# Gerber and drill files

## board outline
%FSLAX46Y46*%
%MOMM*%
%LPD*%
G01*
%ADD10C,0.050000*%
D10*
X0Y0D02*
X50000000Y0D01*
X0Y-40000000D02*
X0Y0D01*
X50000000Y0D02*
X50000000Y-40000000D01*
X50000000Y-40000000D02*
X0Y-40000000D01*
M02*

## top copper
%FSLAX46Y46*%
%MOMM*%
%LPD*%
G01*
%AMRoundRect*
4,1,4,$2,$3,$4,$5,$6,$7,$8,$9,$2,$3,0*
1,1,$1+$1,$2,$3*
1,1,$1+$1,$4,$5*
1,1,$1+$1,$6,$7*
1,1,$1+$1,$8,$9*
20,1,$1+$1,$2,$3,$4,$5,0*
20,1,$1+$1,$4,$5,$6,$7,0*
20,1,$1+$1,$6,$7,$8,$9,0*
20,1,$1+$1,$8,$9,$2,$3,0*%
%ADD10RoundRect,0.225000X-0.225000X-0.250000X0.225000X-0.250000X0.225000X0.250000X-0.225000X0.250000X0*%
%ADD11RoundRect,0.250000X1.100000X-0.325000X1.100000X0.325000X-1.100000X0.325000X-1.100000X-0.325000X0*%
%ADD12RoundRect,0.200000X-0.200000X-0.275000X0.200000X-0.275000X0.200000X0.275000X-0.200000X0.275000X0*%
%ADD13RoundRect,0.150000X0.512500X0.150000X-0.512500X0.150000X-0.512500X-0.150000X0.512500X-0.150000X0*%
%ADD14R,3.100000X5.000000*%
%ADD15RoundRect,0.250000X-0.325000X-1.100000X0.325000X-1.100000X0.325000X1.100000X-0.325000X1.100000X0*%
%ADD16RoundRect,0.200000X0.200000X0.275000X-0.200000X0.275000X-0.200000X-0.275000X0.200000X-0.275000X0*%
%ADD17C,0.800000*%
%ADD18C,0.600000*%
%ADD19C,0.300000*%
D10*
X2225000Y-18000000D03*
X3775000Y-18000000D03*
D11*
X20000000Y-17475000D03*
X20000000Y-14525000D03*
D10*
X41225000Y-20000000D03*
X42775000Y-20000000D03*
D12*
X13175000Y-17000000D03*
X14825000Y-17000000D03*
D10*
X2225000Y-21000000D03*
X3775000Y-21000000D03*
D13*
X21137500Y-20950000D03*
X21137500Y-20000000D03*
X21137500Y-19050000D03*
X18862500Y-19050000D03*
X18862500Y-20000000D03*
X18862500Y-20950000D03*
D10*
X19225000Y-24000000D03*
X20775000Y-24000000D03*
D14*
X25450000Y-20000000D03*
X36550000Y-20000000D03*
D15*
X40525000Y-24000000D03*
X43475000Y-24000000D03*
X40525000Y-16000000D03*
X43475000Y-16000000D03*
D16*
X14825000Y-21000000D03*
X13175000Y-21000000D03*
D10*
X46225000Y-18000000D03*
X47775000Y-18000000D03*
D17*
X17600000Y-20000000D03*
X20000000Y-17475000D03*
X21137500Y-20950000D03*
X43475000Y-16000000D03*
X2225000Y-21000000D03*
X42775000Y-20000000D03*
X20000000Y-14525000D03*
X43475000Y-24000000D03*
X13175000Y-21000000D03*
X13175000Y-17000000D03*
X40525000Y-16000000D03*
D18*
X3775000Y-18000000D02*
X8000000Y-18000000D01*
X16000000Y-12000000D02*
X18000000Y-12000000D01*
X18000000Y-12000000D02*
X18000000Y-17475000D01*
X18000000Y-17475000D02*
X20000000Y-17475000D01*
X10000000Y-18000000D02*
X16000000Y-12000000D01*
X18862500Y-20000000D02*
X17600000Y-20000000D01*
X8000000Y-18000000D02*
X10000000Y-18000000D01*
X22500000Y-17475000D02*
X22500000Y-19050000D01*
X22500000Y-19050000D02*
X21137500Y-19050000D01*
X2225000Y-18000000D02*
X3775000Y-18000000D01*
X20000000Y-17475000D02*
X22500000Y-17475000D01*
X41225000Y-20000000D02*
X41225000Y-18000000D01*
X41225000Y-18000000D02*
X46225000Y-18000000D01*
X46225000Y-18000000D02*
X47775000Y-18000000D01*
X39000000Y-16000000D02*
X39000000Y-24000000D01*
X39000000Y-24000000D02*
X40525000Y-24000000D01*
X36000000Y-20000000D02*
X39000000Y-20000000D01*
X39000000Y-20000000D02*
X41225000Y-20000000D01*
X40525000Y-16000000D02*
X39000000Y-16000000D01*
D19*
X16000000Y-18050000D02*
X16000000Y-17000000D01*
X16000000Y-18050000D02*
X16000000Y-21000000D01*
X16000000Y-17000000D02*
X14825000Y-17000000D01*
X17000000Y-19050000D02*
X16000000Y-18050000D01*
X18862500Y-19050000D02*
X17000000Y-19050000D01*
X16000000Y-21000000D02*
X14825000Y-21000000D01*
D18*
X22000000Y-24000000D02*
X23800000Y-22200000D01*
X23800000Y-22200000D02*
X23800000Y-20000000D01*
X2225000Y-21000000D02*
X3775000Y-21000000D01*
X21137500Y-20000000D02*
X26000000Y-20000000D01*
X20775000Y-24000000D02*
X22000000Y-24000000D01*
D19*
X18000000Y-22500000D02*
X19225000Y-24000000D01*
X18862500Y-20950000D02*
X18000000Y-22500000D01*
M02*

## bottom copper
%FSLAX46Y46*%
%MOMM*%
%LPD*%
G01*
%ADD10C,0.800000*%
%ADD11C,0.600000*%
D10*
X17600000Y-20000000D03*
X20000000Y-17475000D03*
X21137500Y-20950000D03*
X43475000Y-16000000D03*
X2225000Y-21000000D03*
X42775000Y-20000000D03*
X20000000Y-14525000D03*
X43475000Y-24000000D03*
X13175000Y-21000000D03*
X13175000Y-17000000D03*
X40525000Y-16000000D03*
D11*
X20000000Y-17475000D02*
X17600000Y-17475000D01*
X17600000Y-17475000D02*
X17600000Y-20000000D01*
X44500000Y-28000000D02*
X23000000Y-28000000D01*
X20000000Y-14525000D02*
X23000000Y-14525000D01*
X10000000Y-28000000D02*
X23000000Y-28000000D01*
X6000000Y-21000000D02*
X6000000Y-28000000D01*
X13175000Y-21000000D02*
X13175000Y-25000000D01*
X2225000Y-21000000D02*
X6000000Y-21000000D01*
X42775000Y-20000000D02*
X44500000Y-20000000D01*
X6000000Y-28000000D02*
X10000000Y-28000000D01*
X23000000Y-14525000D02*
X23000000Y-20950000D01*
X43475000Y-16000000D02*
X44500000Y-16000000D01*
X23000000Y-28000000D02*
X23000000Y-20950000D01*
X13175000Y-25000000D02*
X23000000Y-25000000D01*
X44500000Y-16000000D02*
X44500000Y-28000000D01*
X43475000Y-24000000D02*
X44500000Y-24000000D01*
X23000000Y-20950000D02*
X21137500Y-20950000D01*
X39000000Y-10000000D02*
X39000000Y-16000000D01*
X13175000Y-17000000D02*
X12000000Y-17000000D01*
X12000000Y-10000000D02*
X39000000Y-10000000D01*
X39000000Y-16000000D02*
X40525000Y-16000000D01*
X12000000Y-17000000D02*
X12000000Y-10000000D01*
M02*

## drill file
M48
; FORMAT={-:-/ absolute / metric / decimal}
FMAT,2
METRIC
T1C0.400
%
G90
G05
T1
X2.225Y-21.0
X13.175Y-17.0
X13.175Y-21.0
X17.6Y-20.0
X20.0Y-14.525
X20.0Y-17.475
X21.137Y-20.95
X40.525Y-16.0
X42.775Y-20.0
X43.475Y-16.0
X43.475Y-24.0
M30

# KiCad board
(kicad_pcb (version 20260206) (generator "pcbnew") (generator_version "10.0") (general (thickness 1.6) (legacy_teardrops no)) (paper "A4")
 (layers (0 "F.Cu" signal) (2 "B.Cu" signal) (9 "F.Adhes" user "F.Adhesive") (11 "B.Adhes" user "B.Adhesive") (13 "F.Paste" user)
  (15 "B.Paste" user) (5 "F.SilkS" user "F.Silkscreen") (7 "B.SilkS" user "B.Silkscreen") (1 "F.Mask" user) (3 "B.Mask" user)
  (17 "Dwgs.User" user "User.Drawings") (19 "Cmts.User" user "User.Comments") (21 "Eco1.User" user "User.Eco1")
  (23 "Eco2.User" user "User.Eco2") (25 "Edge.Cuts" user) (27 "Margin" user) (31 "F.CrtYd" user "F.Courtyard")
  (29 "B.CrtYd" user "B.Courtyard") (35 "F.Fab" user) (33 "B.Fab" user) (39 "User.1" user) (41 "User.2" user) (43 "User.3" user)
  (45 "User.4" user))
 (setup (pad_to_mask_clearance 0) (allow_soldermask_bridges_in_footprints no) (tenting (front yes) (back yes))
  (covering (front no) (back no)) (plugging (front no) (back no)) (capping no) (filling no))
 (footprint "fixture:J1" (layer "F.Cu") (at 3 18)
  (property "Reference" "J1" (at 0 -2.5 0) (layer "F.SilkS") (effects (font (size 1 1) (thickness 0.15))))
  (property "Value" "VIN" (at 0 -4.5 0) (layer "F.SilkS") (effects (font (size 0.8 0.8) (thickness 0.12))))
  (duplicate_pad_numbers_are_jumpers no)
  (pad "1" smd roundrect (at -0.775 0) (size 0.9 0.95) (layers "F.Cu" "F.Mask" "F.Paste") (roundrect_rratio 0.25) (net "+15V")
   (thermal_bridge_angle 45))
  (pad "2" smd roundrect (at 0.775 0) (size 0.9 0.95) (layers "F.Cu" "F.Mask" "F.Paste") (roundrect_rratio 0.25) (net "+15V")
   (thermal_bridge_angle 45)))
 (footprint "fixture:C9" (layer "F.Cu") (at 20 16 90)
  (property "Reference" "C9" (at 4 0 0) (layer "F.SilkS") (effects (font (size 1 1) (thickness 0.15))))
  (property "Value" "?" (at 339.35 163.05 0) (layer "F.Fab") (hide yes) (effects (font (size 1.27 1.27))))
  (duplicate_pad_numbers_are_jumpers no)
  (pad "1" smd roundrect (at -1.475 0 90) (size 1.15 2.7) (layers "F.Cu" "F.Mask" "F.Paste") (roundrect_rratio 0.217391) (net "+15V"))
  (pad "2" smd roundrect (at 1.475 0 90) (size 1.15 2.7) (layers "F.Cu" "F.Mask" "F.Paste") (roundrect_rratio 0.217391) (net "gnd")))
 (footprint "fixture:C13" (layer "F.Cu") (at 42 20)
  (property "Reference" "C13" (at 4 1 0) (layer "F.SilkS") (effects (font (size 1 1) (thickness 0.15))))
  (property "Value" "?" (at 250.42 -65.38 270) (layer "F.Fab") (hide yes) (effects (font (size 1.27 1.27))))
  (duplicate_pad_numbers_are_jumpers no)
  (pad "1" smd roundrect (at -0.775 0) (size 0.9 0.95) (layers "F.Cu" "F.Mask" "F.Paste") (roundrect_rratio 0.25) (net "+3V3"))
  (pad "2" smd roundrect (at 0.775 0) (size 0.9 0.95) (layers "F.Cu" "F.Mask" "F.Paste") (roundrect_rratio 0.25) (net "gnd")))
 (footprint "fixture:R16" (layer "F.Cu") (at 14 17)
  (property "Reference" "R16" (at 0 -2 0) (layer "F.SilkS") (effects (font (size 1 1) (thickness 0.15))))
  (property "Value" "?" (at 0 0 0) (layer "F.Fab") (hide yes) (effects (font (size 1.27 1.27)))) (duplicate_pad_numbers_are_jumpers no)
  (pad "1" smd roundrect (at -0.825 0) (size 0.8 0.95) (layers "F.Cu" "F.Mask" "F.Paste") (roundrect_rratio 0.25) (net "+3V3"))
  (pad "2" smd roundrect (at 0.825 0) (size 0.8 0.95) (layers "F.Cu" "F.Mask" "F.Paste") (roundrect_rratio 0.25) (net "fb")))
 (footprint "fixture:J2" (layer "F.Cu") (at 3 21)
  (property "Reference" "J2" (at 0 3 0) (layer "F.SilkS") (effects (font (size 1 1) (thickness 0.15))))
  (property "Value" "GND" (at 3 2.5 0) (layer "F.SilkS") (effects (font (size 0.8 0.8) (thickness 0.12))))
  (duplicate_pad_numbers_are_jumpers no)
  (pad "1" smd roundrect (at -0.775 0) (size 0.9 0.95) (layers "F.Cu" "F.Mask" "F.Paste") (roundrect_rratio 0.25) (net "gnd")
   (thermal_bridge_angle 45))
  (pad "2" smd roundrect (at 0.775 0) (size 0.9 0.95) (layers "F.Cu" "F.Mask" "F.Paste") (roundrect_rratio 0.25) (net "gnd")
   (thermal_bridge_angle 45)))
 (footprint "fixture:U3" (layer "F.Cu") (at 20 20 180)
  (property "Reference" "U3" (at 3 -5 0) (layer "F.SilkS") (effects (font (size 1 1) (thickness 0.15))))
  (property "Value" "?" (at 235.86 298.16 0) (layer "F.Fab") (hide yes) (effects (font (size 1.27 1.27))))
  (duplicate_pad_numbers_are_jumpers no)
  (pad "1" smd roundrect (at -1.1375 -0.95 180) (size 1.325 0.6) (layers "F.Cu" "F.Mask" "F.Paste") (roundrect_rratio 0.25) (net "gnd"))
  (pad "2" smd roundrect (at -1.1375 0 180) (size 1.325 0.6) (layers "F.Cu" "F.Mask" "F.Paste") (roundrect_rratio 0.25) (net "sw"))
  (pad "3" smd roundrect (at -1.1375 0.95 180) (size 1.325 0.6) (layers "F.Cu" "F.Mask" "F.Paste") (roundrect_rratio 0.25) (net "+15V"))
  (pad "4" smd roundrect (at 1.1375 0.95 180) (size 1.325 0.6) (layers "F.Cu" "F.Mask" "F.Paste") (roundrect_rratio 0.25) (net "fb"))
  (pad "5" smd roundrect (at 1.1375 0 180) (size 1.325 0.6) (layers "F.Cu" "F.Mask" "F.Paste") (roundrect_rratio 0.25) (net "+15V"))
  (pad "6" smd roundrect (at 1.1375 -0.95 180) (size 1.325 0.6) (layers "F.Cu" "F.Mask" "F.Paste") (roundrect_rratio 0.25) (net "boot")))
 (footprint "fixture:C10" (layer "F.Cu") (at 20 24)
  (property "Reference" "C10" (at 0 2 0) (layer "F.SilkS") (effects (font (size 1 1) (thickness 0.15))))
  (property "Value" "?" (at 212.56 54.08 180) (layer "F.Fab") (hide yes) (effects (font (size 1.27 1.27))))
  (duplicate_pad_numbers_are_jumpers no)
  (pad "1" smd roundrect (at -0.775 0) (size 0.9 0.95) (layers "F.Cu" "F.Mask" "F.Paste") (roundrect_rratio 0.25) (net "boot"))
  (pad "2" smd roundrect (at 0.775 0) (size 0.9 0.95) (layers "F.Cu" "F.Mask" "F.Paste") (roundrect_rratio 0.25) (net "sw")))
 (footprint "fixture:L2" (layer "F.Cu") (at 31 20)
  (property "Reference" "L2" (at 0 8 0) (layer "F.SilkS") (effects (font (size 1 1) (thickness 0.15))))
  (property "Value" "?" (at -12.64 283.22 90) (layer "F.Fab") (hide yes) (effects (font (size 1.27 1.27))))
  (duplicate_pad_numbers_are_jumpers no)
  (pad "1" smd rect (at -5.55 0) (size 3.1 5) (layers "F.Cu" "F.Mask" "F.Paste") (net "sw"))
  (pad "2" smd rect (at 5.55 0) (size 3.1 5) (layers "F.Cu" "F.Mask" "F.Paste") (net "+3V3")))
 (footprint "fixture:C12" (layer "F.Cu") (at 42 24)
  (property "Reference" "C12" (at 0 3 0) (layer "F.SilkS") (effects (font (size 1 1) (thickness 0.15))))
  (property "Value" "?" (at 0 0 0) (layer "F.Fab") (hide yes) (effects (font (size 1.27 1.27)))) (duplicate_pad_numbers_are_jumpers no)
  (pad "1" smd roundrect (at -1.475 0) (size 1.15 2.7) (layers "F.Cu" "F.Mask" "F.Paste") (roundrect_rratio 0.217391) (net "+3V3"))
  (pad "2" smd roundrect (at 1.475 0) (size 1.15 2.7) (layers "F.Cu" "F.Mask" "F.Paste") (roundrect_rratio 0.217391) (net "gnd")))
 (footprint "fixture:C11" (layer "F.Cu") (at 42 16)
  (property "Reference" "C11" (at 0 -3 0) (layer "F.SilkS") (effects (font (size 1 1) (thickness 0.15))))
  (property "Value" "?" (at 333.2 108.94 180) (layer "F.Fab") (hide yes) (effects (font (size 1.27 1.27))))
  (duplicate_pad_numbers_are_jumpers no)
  (pad "1" smd roundrect (at -1.475 0) (size 1.15 2.7) (layers "F.Cu" "F.Mask" "F.Paste") (roundrect_rratio 0.217391) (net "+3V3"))
  (pad "2" smd roundrect (at 1.475 0) (size 1.15 2.7) (layers "F.Cu" "F.Mask" "F.Paste") (roundrect_rratio 0.217391) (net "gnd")))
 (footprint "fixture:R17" (layer "F.Cu") (at 14 21 180)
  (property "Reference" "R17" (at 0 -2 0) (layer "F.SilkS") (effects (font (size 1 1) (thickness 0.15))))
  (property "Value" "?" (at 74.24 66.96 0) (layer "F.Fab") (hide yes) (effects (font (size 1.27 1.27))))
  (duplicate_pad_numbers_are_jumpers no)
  (pad "1" smd roundrect (at -0.825 0 180) (size 0.8 0.95) (layers "F.Cu" "F.Mask" "F.Paste") (roundrect_rratio 0.25) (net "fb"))
  (pad "2" smd roundrect (at 0.825 0 180) (size 0.8 0.95) (layers "F.Cu" "F.Mask" "F.Paste") (roundrect_rratio 0.25) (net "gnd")))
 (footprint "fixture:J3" (layer "F.Cu") (at 47 18)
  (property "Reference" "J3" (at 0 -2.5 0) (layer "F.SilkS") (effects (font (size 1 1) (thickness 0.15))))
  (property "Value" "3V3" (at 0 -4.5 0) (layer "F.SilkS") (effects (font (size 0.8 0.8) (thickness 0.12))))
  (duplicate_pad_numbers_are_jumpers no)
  (pad "1" smd roundrect (at -0.775 0) (size 0.9 0.95) (layers "F.Cu" "F.Mask" "F.Paste") (roundrect_rratio 0.25) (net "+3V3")
   (thermal_bridge_angle 45))
  (pad "2" smd roundrect (at 0.775 0) (size 0.9 0.95) (layers "F.Cu" "F.Mask" "F.Paste") (roundrect_rratio 0.25) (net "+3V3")
   (thermal_bridge_angle 45)))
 (gr_line (start 0 0) (end 50 0) (stroke (width 0.05) (type default)) (layer "Edge.Cuts"))
 (gr_line (start 0 40) (end 0 0) (stroke (width 0.05) (type default)) (layer "Edge.Cuts"))
 (gr_line (start 50 0) (end 50 40) (stroke (width 0.05) (type default)) (layer "Edge.Cuts"))
 (gr_line (start 50 40) (end 0 40) (stroke (width 0.05) (type default)) (layer "Edge.Cuts"))
 (segment (start 3.775 18) (end 8 18) (width 0.6) (layer "F.Cu") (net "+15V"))
 (segment (start 16 12) (end 18 12) (width 0.6) (layer "F.Cu") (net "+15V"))
 (segment (start 18 12) (end 18 17.475) (width 0.6) (layer "F.Cu") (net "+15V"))
 (segment (start 18 17.475) (end 20 17.475) (width 0.6) (layer "F.Cu") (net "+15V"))
 (segment (start 10 18) (end 16 12) (width 0.6) (layer "F.Cu") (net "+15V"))
 (segment (start 18.8625 20) (end 17.6 20) (width 0.6) (layer "F.Cu") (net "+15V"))
 (segment (start 8 18) (end 10 18) (width 0.6) (layer "F.Cu") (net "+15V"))
 (segment (start 22.5 17.475) (end 22.5 19.05) (width 0.6) (layer "F.Cu") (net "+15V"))
 (segment (start 22.5 19.05) (end 21.1375 19.05) (width 0.6) (layer "F.Cu") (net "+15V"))
 (segment (start 2.225 18) (end 3.775 18) (width 0.6) (layer "F.Cu") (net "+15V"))
 (segment (start 20 17.475) (end 22.5 17.475) (width 0.6) (layer "F.Cu") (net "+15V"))
 (via (at 17.6 20) (size 0.8) (drill 0.4) (layers "F.Cu" "B.Cu") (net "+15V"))
 (via (at 20 17.475) (size 0.8) (drill 0.4) (layers "F.Cu" "B.Cu") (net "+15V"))
 (segment (start 20 17.475) (end 17.6 17.475) (width 0.6) (layer "B.Cu") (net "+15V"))
 (segment (start 17.6 17.475) (end 17.6 20) (width 0.6) (layer "B.Cu") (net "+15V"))
 (via (at 21.1375 20.95) (size 0.8) (drill 0.4) (layers "F.Cu" "B.Cu") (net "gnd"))
 (via (at 43.475 16) (size 0.8) (drill 0.4) (layers "F.Cu" "B.Cu") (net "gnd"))
 (via (at 2.225 21) (size 0.8) (drill 0.4) (layers "F.Cu" "B.Cu") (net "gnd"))
 (via (at 42.775 20) (size 0.8) (drill 0.4) (layers "F.Cu" "B.Cu") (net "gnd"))
 (via (at 20 14.525) (size 0.8) (drill 0.4) (layers "F.Cu" "B.Cu") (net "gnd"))
 (via (at 43.475 24) (size 0.8) (drill 0.4) (layers "F.Cu" "B.Cu") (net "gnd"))
 (via (at 13.175 21) (size 0.8) (drill 0.4) (layers "F.Cu" "B.Cu") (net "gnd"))
 (segment (start 44.5 28) (end 23 28) (width 0.6) (layer "B.Cu") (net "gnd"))
 (segment (start 20 14.525) (end 23 14.525) (width 0.6) (layer "B.Cu") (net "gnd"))
 (segment (start 10 28) (end 23 28) (width 0.6) (layer "B.Cu") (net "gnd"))
 (segment (start 6 21) (end 6 28) (width 0.6) (layer "B.Cu") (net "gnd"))
 (segment (start 13.175 21) (end 13.175 25) (width 0.6) (layer "B.Cu") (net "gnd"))
 (segment (start 2.225 21) (end 6 21) (width 0.6) (layer "B.Cu") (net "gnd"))
 (segment (start 42.775 20) (end 44.5 20) (width 0.6) (layer "B.Cu") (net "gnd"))
 (segment (start 6 28) (end 10 28) (width 0.6) (layer "B.Cu") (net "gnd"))
 (segment (start 23 14.525) (end 23 20.95) (width 0.6) (layer "B.Cu") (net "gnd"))
 (segment (start 43.475 16) (end 44.5 16) (width 0.6) (layer "B.Cu") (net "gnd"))
 (segment (start 23 28) (end 23 20.95) (width 0.6) (layer "B.Cu") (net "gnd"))
 (segment (start 13.175 25) (end 23 25) (width 0.6) (layer "B.Cu") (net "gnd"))
 (segment (start 44.5 16) (end 44.5 28) (width 0.6) (layer "B.Cu") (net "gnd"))
 (segment (start 43.475 24) (end 44.5 24) (width 0.6) (layer "B.Cu") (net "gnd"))
 (segment (start 23 20.95) (end 21.1375 20.95) (width 0.6) (layer "B.Cu") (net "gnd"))
 (segment (start 41.225 20) (end 41.225 18) (width 0.6) (layer "F.Cu") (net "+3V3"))
 (segment (start 41.225 18) (end 46.225 18) (width 0.6) (layer "F.Cu") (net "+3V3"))
 (segment (start 46.225 18) (end 47.775 18) (width 0.6) (layer "F.Cu") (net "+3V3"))
 (segment (start 39 16) (end 39 24) (width 0.6) (layer "F.Cu") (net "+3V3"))
 (segment (start 39 24) (end 40.525 24) (width 0.6) (layer "F.Cu") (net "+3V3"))
 (segment (start 36 20) (end 39 20) (width 0.6) (layer "F.Cu") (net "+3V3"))
 (segment (start 39 20) (end 41.225 20) (width 0.6) (layer "F.Cu") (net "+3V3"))
 (segment (start 40.525 16) (end 39 16) (width 0.6) (layer "F.Cu") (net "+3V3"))
 (via (at 13.175 17) (size 0.8) (drill 0.4) (layers "F.Cu" "B.Cu") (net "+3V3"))
 (via (at 40.525 16) (size 0.8) (drill 0.4) (layers "F.Cu" "B.Cu") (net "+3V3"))
 (segment (start 39 10) (end 39 16) (width 0.6) (layer "B.Cu") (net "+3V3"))
 (segment (start 13.175 17) (end 12 17) (width 0.6) (layer "B.Cu") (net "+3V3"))
 (segment (start 12 10) (end 39 10) (width 0.6) (layer "B.Cu") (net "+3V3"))
 (segment (start 39 16) (end 40.525 16) (width 0.6) (layer "B.Cu") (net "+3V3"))
 (segment (start 12 17) (end 12 10) (width 0.6) (layer "B.Cu") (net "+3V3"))
 (segment (start 16 18.05) (end 16 17) (width 0.3) (layer "F.Cu") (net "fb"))
 (segment (start 16 18.05) (end 16 21) (width 0.3) (layer "F.Cu") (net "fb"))
 (segment (start 16 17) (end 14.825 17) (width 0.3) (layer "F.Cu") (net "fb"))
 (segment (start 17 19.05) (end 16 18.05) (width 0.3) (layer "F.Cu") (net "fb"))
 (segment (start 18.8625 19.05) (end 17 19.05) (width 0.3) (layer "F.Cu") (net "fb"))
 (segment (start 16 21) (end 14.825 21) (width 0.3) (layer "F.Cu") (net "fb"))
 (segment (start 22 24) (end 23.8 22.2) (width 0.6) (layer "F.Cu") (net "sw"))
 (segment (start 23.8 22.2) (end 23.8 20) (width 0.6) (layer "F.Cu") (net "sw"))
 (segment (start 2.225 21) (end 3.775 21) (width 0.6) (layer "F.Cu") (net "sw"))
 (segment (start 21.1375 20) (end 26 20) (width 0.6) (layer "F.Cu") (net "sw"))
 (segment (start 20.775 24) (end 22 24) (width 0.6) (layer "F.Cu") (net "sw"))
 (segment (start 18 22.5) (end 19.225 24) (width 0.3) (layer "F.Cu") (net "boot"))
 (segment (start 18.8625 20.95) (end 18 22.5) (width 0.3) (layer "F.Cu") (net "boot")))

